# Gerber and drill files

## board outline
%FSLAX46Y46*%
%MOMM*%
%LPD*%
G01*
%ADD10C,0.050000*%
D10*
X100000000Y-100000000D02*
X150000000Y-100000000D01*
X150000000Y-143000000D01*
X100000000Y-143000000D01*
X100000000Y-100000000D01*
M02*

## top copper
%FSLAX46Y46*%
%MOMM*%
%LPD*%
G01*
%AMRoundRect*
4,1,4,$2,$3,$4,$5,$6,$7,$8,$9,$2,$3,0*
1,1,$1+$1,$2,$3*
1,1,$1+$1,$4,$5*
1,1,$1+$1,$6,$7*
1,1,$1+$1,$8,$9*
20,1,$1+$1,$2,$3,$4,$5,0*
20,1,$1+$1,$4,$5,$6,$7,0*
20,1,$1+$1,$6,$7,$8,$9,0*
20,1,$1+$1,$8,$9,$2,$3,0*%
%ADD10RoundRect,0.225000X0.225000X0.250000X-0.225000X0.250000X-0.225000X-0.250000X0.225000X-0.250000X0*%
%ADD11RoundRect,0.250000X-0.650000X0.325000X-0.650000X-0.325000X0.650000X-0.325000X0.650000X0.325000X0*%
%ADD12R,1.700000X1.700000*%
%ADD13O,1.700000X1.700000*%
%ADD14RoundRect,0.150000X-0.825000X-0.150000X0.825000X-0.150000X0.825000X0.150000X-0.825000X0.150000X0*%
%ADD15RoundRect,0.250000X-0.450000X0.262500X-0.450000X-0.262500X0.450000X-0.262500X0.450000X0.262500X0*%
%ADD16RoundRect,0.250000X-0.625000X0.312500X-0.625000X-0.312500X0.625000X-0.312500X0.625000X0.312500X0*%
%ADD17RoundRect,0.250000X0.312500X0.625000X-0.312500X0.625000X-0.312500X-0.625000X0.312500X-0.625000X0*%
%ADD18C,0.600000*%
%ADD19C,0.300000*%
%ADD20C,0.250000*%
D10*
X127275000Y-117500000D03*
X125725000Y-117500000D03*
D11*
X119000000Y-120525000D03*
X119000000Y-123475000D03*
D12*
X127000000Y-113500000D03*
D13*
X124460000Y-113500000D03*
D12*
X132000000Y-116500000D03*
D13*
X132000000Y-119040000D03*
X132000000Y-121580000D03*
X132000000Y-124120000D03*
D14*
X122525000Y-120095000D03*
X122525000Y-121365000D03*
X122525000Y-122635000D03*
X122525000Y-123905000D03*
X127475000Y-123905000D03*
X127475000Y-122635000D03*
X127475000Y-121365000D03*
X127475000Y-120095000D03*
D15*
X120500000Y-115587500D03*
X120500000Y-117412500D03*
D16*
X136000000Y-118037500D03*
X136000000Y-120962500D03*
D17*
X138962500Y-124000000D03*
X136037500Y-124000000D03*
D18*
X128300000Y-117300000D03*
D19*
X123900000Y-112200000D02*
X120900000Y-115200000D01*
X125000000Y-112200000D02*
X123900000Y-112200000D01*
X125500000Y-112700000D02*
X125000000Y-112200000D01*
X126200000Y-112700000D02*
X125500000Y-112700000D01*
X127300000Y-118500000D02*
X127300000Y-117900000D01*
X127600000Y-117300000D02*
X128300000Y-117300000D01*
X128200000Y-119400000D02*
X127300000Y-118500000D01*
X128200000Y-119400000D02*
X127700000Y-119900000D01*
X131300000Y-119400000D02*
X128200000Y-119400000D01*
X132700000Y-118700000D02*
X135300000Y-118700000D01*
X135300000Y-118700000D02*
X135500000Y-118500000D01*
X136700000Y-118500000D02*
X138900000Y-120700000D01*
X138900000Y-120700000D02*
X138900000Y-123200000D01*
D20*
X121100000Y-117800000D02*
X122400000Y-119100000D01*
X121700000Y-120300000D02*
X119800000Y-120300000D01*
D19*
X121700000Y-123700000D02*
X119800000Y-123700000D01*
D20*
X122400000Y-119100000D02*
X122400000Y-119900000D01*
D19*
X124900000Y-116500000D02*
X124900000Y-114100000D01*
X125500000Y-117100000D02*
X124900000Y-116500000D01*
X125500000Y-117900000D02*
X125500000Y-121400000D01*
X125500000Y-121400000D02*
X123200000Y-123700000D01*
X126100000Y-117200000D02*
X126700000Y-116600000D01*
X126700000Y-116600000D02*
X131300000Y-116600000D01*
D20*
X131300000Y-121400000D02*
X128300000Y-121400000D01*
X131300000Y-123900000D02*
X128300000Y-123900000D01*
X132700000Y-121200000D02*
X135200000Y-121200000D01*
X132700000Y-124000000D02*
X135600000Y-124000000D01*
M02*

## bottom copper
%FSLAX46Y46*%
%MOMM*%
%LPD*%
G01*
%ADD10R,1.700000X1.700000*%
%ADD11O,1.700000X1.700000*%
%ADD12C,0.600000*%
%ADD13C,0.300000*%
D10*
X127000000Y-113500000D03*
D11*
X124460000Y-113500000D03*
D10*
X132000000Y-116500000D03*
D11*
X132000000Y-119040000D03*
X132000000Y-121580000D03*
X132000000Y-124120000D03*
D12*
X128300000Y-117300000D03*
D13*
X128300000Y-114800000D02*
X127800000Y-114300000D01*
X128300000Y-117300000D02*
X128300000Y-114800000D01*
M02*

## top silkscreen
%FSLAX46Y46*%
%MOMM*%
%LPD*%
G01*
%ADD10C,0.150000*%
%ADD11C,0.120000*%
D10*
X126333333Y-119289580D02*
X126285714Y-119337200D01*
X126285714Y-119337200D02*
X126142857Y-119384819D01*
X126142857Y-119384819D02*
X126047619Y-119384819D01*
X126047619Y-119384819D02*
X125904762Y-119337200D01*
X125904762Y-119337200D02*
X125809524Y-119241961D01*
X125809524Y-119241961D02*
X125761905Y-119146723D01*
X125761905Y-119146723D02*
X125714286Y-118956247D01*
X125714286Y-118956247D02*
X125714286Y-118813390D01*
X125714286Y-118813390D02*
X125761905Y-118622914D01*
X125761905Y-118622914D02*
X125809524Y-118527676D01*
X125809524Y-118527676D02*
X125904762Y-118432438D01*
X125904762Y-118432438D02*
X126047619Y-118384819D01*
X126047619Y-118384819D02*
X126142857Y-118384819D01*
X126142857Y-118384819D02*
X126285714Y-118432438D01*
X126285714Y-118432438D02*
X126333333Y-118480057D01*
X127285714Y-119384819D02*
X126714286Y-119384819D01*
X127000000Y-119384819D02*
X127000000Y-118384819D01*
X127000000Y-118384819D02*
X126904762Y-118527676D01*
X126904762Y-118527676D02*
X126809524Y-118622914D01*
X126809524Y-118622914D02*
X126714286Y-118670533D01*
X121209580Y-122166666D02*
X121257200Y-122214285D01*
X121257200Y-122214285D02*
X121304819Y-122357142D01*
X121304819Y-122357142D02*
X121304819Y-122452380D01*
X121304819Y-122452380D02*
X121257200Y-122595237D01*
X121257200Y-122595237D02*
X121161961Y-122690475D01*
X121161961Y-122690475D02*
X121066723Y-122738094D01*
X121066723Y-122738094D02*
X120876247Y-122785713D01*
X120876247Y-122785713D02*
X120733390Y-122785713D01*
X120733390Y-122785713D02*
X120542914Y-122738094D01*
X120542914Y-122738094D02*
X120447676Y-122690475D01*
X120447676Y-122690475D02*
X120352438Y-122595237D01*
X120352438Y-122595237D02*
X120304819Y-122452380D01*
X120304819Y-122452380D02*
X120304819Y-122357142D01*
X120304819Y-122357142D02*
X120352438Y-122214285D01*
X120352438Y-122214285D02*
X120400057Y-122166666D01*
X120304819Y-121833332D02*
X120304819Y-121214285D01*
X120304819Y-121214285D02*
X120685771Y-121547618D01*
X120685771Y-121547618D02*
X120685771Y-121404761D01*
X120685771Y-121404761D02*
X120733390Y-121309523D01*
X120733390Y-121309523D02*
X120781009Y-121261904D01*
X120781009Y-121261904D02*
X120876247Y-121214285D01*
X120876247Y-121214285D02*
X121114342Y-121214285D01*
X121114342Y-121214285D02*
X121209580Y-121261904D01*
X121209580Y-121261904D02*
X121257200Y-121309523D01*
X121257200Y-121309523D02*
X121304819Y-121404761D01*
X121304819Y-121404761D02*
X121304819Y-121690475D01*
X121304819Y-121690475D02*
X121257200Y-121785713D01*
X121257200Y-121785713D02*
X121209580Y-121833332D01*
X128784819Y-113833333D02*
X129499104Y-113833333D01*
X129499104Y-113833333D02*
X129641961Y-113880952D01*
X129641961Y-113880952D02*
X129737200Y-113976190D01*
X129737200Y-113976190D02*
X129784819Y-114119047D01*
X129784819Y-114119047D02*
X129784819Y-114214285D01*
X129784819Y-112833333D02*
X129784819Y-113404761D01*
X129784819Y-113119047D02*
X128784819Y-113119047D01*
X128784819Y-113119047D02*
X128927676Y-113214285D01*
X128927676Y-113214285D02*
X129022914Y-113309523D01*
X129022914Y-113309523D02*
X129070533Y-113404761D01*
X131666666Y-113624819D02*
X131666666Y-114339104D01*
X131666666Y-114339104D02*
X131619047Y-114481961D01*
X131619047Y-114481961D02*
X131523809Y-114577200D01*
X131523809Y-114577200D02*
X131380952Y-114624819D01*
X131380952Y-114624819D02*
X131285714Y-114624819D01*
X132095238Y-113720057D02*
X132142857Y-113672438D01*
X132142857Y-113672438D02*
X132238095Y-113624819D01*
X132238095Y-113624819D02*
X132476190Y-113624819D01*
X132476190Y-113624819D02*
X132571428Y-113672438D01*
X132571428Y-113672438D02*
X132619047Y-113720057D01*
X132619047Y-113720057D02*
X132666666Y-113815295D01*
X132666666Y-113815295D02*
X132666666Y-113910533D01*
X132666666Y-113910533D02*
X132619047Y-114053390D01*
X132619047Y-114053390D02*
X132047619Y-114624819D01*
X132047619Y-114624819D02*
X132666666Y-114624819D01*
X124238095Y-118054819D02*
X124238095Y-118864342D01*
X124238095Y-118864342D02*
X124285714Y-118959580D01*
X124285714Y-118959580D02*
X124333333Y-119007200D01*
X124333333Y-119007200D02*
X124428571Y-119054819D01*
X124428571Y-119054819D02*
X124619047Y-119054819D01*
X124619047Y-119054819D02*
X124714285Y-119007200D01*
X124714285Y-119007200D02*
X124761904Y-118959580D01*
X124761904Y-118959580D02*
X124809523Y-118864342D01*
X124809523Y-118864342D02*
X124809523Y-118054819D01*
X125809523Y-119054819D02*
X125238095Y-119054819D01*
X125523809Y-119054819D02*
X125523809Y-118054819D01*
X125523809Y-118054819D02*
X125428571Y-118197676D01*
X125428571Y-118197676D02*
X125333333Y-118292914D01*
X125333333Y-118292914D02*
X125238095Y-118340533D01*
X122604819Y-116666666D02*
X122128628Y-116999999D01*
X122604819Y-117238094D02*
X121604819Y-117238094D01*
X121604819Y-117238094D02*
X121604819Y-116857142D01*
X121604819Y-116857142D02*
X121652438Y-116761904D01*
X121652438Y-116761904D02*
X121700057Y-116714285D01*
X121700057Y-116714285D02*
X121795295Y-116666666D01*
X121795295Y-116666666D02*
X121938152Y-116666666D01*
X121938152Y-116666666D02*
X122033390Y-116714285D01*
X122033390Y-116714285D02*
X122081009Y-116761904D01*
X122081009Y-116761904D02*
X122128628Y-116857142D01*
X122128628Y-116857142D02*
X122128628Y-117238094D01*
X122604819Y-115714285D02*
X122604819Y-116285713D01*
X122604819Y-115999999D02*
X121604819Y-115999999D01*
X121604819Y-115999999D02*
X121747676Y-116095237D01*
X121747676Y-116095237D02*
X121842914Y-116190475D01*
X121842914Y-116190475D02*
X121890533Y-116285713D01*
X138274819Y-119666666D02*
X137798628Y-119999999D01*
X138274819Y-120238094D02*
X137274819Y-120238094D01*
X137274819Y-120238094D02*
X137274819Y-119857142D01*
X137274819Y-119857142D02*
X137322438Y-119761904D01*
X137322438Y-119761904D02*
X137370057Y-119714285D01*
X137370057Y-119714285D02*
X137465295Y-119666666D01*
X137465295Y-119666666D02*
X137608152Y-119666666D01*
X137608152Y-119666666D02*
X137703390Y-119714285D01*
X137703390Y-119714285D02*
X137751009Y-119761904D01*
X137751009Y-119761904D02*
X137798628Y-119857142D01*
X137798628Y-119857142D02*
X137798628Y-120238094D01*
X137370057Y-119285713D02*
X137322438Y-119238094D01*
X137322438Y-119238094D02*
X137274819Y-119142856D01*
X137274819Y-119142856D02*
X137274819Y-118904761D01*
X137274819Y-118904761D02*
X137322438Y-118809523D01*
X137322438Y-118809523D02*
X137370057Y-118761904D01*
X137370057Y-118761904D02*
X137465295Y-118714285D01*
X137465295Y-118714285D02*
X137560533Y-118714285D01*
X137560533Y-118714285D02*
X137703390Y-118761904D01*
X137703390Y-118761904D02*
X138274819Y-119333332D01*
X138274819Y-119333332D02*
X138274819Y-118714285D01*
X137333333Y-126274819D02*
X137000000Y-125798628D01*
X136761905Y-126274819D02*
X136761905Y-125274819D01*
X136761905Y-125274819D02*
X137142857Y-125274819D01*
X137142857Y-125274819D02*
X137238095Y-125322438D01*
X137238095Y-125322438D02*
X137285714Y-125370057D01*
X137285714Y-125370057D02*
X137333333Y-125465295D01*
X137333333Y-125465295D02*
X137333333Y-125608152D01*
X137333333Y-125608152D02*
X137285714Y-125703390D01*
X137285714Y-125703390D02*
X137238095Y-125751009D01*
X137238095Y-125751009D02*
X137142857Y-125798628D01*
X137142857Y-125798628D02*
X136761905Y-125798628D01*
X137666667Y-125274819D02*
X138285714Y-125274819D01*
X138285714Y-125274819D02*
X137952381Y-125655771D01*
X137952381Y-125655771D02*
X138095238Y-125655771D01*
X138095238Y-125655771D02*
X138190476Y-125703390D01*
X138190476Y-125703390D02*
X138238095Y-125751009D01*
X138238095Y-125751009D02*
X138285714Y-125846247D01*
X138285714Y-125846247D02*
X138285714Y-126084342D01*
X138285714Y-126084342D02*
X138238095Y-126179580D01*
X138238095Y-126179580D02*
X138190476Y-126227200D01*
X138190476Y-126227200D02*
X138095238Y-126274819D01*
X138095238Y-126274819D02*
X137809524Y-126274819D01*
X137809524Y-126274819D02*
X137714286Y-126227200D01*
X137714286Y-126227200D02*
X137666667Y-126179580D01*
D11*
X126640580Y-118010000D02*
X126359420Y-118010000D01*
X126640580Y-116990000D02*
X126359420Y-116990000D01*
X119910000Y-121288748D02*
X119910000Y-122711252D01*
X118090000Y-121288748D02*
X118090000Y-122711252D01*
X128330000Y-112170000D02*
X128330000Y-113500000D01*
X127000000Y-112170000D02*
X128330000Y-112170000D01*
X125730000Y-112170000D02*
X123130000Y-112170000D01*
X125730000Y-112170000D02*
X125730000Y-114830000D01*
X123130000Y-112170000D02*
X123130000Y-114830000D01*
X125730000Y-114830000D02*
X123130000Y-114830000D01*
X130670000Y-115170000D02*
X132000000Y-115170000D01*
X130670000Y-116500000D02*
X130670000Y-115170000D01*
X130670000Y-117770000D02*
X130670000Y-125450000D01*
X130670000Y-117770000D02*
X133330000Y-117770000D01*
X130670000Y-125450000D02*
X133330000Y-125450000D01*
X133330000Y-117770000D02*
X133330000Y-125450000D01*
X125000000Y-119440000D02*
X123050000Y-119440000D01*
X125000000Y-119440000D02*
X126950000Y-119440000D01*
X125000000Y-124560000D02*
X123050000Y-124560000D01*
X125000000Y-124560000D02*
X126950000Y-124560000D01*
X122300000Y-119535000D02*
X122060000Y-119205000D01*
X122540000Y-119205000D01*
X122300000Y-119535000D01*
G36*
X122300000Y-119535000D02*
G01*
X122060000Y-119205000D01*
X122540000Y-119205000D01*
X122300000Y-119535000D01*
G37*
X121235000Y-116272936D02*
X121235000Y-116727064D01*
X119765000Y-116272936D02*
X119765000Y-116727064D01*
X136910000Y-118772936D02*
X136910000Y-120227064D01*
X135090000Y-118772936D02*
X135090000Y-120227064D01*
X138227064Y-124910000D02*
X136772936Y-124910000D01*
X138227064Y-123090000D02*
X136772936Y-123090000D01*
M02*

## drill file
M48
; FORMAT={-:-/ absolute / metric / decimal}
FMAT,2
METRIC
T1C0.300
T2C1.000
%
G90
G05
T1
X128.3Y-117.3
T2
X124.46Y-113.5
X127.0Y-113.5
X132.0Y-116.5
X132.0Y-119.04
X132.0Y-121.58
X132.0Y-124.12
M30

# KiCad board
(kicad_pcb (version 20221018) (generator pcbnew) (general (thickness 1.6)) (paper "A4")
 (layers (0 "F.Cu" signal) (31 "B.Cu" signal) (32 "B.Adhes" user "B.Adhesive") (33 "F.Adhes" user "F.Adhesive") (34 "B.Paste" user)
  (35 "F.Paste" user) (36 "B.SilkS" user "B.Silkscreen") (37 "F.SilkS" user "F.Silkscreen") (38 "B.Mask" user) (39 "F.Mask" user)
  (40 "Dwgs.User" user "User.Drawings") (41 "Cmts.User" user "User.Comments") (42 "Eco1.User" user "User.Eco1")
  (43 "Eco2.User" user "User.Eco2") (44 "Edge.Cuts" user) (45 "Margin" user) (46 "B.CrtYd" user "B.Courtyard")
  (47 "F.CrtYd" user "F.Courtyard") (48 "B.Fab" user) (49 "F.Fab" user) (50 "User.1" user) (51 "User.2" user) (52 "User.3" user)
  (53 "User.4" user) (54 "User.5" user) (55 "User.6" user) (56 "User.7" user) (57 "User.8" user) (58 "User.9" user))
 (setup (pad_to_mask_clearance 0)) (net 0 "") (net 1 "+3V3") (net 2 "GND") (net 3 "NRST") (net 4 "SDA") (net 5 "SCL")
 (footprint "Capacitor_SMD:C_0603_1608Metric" (layer "F.Cu") (at 126.5 117.5 180)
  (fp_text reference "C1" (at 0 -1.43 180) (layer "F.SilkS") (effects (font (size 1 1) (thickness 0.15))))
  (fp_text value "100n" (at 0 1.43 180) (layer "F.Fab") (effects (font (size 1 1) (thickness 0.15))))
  (fp_line (start -0.14058 -0.51) (end 0.14058 -0.51) (stroke (width 0.12) (type solid)) (layer "F.SilkS"))
  (fp_line (start -0.14058 0.51) (end 0.14058 0.51) (stroke (width 0.12) (type solid)) (layer "F.SilkS"))
  (pad "1" smd roundrect (at -0.775 0 180) (size 0.9 0.95) (layers "F.Cu" "F.Paste" "F.Mask") (roundrect_rratio 0.25) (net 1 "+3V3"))
  (pad "2" smd roundrect (at 0.775 0 180) (size 0.9 0.95) (layers "F.Cu" "F.Paste" "F.Mask") (roundrect_rratio 0.25) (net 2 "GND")))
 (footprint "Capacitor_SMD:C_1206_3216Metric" (layer "F.Cu") (at 119 122 -90)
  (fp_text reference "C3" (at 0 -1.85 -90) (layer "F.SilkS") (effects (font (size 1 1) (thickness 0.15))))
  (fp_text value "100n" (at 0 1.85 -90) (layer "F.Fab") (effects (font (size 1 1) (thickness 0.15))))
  (fp_line (start -0.711252 -0.91) (end 0.711252 -0.91) (stroke (width 0.12) (type solid)) (layer "F.SilkS"))
  (fp_line (start -0.711252 0.91) (end 0.711252 0.91) (stroke (width 0.12) (type solid)) (layer "F.SilkS"))
  (pad "1" smd roundrect (at -1.475 0 270) (size 1.15 1.8) (layers "F.Cu" "F.Paste" "F.Mask") (roundrect_rratio 0.217391) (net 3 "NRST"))
  (pad "2" smd roundrect (at 1.475 0 270) (size 1.15 1.8) (layers "F.Cu" "F.Paste" "F.Mask") (roundrect_rratio 0.217391) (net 2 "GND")))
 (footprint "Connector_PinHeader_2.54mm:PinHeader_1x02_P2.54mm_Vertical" (layer "F.Cu") (at 127 113.5 -90)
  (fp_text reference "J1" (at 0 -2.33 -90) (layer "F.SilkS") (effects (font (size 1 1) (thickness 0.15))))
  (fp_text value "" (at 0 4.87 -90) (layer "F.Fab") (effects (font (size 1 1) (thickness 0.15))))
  (fp_line (start -1.33 -1.33) (end 0 -1.33) (stroke (width 0.12) (type solid)) (layer "F.SilkS"))
  (fp_line (start -1.33 0) (end -1.33 -1.33) (stroke (width 0.12) (type solid)) (layer "F.SilkS"))
  (fp_line (start -1.33 1.27) (end -1.33 3.87) (stroke (width 0.12) (type solid)) (layer "F.SilkS"))
  (fp_line (start -1.33 1.27) (end 1.33 1.27) (stroke (width 0.12) (type solid)) (layer "F.SilkS"))
  (fp_line (start -1.33 3.87) (end 1.33 3.87) (stroke (width 0.12) (type solid)) (layer "F.SilkS"))
  (fp_line (start 1.33 1.27) (end 1.33 3.87) (stroke (width 0.12) (type solid)) (layer "F.SilkS"))
  (pad "1" thru_hole rect (at 0 0 270) (size 1.7 1.7) (drill 1) (layers "*.Cu" "*.Mask") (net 1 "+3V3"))
  (pad "2" thru_hole oval (at 0 2.54 270) (size 1.7 1.7) (drill 1) (layers "*.Cu" "*.Mask") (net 2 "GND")))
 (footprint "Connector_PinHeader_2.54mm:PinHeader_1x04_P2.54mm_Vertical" (layer "F.Cu") (at 132 116.5)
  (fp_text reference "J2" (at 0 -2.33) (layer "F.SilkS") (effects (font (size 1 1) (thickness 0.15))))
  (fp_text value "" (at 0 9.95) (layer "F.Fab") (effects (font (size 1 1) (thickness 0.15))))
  (fp_line (start -1.33 -1.33) (end 0 -1.33) (stroke (width 0.12) (type solid)) (layer "F.SilkS"))
  (fp_line (start -1.33 0) (end -1.33 -1.33) (stroke (width 0.12) (type solid)) (layer "F.SilkS"))
  (fp_line (start -1.33 1.27) (end -1.33 8.95) (stroke (width 0.12) (type solid)) (layer "F.SilkS"))
  (fp_line (start -1.33 1.27) (end 1.33 1.27) (stroke (width 0.12) (type solid)) (layer "F.SilkS"))
  (fp_line (start -1.33 8.95) (end 1.33 8.95) (stroke (width 0.12) (type solid)) (layer "F.SilkS"))
  (fp_line (start 1.33 1.27) (end 1.33 8.95) (stroke (width 0.12) (type solid)) (layer "F.SilkS"))
  (pad "1" thru_hole rect (at 0 0) (size 1.7 1.7) (drill 1) (layers "*.Cu" "*.Mask") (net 2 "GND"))
  (pad "2" thru_hole oval (at 0 2.54) (size 1.7 1.7) (drill 1) (layers "*.Cu" "*.Mask") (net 1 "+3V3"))
  (pad "3" thru_hole oval (at 0 5.08) (size 1.7 1.7) (drill 1) (layers "*.Cu" "*.Mask") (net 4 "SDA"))
  (pad "4" thru_hole oval (at 0 7.62) (size 1.7 1.7) (drill 1) (layers "*.Cu" "*.Mask") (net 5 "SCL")))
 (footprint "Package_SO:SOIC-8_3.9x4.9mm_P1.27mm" (layer "F.Cu") (at 125 122)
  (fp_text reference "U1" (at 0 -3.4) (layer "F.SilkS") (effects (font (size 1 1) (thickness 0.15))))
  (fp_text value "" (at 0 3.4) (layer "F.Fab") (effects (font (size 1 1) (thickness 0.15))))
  (fp_line (start 0 -2.56) (end -1.95 -2.56) (stroke (width 0.12) (type solid)) (layer "F.SilkS"))
  (fp_line (start 0 -2.56) (end 1.95 -2.56) (stroke (width 0.12) (type solid)) (layer "F.SilkS"))
  (fp_line (start 0 2.56) (end -1.95 2.56) (stroke (width 0.12) (type solid)) (layer "F.SilkS"))
  (fp_line (start 0 2.56) (end 1.95 2.56) (stroke (width 0.12) (type solid)) (layer "F.SilkS"))
  (fp_poly
   (pts (xy -2.7 -2.465) (xy -2.94 -2.795) (xy -2.46 -2.795) (xy -2.7 -2.465)) (stroke (width 0.12) (type solid)) (fill solid)
   (layer "F.SilkS"))
  (pad "1" smd roundrect (at -2.475 -1.905) (size 1.95 0.6) (layers "F.Cu" "F.Paste" "F.Mask") (roundrect_rratio 0.25) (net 3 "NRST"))
  (pad "2" smd roundrect (at -2.475 -0.635) (size 1.95 0.6) (layers "F.Cu" "F.Paste" "F.Mask") (roundrect_rratio 0.25))
  (pad "3" smd roundrect (at -2.475 0.635) (size 1.95 0.6) (layers "F.Cu" "F.Paste" "F.Mask") (roundrect_rratio 0.25))
  (pad "4" smd roundrect (at -2.475 1.905) (size 1.95 0.6) (layers "F.Cu" "F.Paste" "F.Mask") (roundrect_rratio 0.25) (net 2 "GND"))
  (pad "5" smd roundrect (at 2.475 1.905) (size 1.95 0.6) (layers "F.Cu" "F.Paste" "F.Mask") (roundrect_rratio 0.25) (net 5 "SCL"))
  (pad "6" smd roundrect (at 2.475 0.635) (size 1.95 0.6) (layers "F.Cu" "F.Paste" "F.Mask") (roundrect_rratio 0.25))
  (pad "7" smd roundrect (at 2.475 -0.635) (size 1.95 0.6) (layers "F.Cu" "F.Paste" "F.Mask") (roundrect_rratio 0.25) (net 4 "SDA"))
  (pad "8" smd roundrect (at 2.475 -1.905) (size 1.95 0.6) (layers "F.Cu" "F.Paste" "F.Mask") (roundrect_rratio 0.25) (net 1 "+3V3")))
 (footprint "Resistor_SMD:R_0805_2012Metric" (layer "F.Cu") (at 120.5 116.5 -90)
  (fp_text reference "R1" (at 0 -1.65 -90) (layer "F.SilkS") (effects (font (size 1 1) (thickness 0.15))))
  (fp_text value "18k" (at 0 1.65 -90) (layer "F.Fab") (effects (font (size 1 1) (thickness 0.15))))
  (fp_line (start -0.227064 -0.735) (end 0.227064 -0.735) (stroke (width 0.12) (type solid)) (layer "F.SilkS"))
  (fp_line (start -0.227064 0.735) (end 0.227064 0.735) (stroke (width 0.12) (type solid)) (layer "F.SilkS"))
  (pad "1" smd roundrect (at -0.9125 0 270) (size 1.025 1.4) (layers "F.Cu" "F.Paste" "F.Mask") (roundrect_rratio 0.243902) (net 1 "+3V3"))
  (pad "2" smd roundrect (at 0.9125 0 270) (size 1.025 1.4) (layers "F.Cu" "F.Paste" "F.Mask") (roundrect_rratio 0.243902) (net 3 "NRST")))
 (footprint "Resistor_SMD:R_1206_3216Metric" (layer "F.Cu") (at 136 119.5 -90)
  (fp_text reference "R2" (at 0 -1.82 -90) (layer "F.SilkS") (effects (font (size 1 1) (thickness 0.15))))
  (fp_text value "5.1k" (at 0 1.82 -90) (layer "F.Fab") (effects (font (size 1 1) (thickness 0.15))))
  (fp_line (start -0.727064 -0.91) (end 0.727064 -0.91) (stroke (width 0.12) (type solid)) (layer "F.SilkS"))
  (fp_line (start -0.727064 0.91) (end 0.727064 0.91) (stroke (width 0.12) (type solid)) (layer "F.SilkS"))
  (pad "1" smd roundrect (at -1.4625 0 270) (size 1.125 1.75) (layers "F.Cu" "F.Paste" "F.Mask") (roundrect_rratio 0.222222) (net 1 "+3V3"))
  (pad "2" smd roundrect (at 1.4625 0 270) (size 1.125 1.75) (layers "F.Cu" "F.Paste" "F.Mask") (roundrect_rratio 0.222222) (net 4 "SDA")))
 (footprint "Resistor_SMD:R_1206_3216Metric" (layer "F.Cu") (at 137.5 124 180)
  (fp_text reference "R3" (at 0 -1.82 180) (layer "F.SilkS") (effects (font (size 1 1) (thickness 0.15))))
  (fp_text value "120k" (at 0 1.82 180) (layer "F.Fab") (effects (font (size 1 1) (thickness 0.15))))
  (fp_line (start -0.727064 -0.91) (end 0.727064 -0.91) (stroke (width 0.12) (type solid)) (layer "F.SilkS"))
  (fp_line (start -0.727064 0.91) (end 0.727064 0.91) (stroke (width 0.12) (type solid)) (layer "F.SilkS"))
  (pad "1" smd roundrect (at -1.4625 0 180) (size 1.125 1.75) (layers "F.Cu" "F.Paste" "F.Mask") (roundrect_rratio 0.222222) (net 1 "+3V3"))
  (pad "2" smd roundrect (at 1.4625 0 180) (size 1.125 1.75) (layers "F.Cu" "F.Paste" "F.Mask") (roundrect_rratio 0.222222) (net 5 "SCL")))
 (gr_rect (start 100 100) (end 150 143) (stroke (width 0.05) (type default)) (fill none) (layer "Edge.Cuts"))
 (segment (start 123.9 112.2) (end 120.9 115.2) (width 0.3) (layer "F.Cu") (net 1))
 (segment (start 125 112.2) (end 123.9 112.2) (width 0.3) (layer "F.Cu") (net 1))
 (segment (start 125.5 112.7) (end 125 112.2) (width 0.3) (layer "F.Cu") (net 1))
 (segment (start 126.2 112.7) (end 125.5 112.7) (width 0.3) (layer "F.Cu") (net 1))
 (segment (start 127.3 118.5) (end 127.3 117.9) (width 0.3) (layer "F.Cu") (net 1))
 (segment (start 127.6 117.3) (end 128.3 117.3) (width 0.3) (layer "F.Cu") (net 1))
 (segment (start 128.2 119.4) (end 127.3 118.5) (width 0.3) (layer "F.Cu") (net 1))
 (segment (start 128.2 119.4) (end 127.7 119.9) (width 0.3) (layer "F.Cu") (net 1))
 (segment (start 131.3 119.4) (end 128.2 119.4) (width 0.3) (layer "F.Cu") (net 1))
 (segment (start 132.7 118.7) (end 135.3 118.7) (width 0.3) (layer "F.Cu") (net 1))
 (segment (start 135.3 118.7) (end 135.5 118.5) (width 0.3) (layer "F.Cu") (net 1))
 (segment (start 136.7 118.5) (end 138.9 120.7) (width 0.3) (layer "F.Cu") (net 1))
 (segment (start 138.9 120.7) (end 138.9 123.2) (width 0.3) (layer "F.Cu") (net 1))
 (via (at 128.3 117.3) (size 0.6) (drill 0.3) (layers "F.Cu" "B.Cu") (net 1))
 (segment (start 121.1 117.8) (end 122.4 119.1) (width 0.25) (layer "F.Cu") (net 3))
 (segment (start 121.7 120.3) (end 119.8 120.3) (width 0.25) (layer "F.Cu") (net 3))
 (segment (start 121.7 123.7) (end 119.8 123.7) (width 0.3) (layer "F.Cu") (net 2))
 (segment (start 122.4 119.1) (end 122.4 119.9) (width 0.25) (layer "F.Cu") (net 3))
 (segment (start 124.9 116.5) (end 124.9 114.1) (width 0.3) (layer "F.Cu") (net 2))
 (segment (start 125.5 117.1) (end 124.9 116.5) (width 0.3) (layer "F.Cu") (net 2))
 (segment (start 125.5 117.9) (end 125.5 121.4) (width 0.3) (layer "F.Cu") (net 2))
 (segment (start 125.5 121.4) (end 123.2 123.7) (width 0.3) (layer "F.Cu") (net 2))
 (segment (start 126.1 117.2) (end 126.7 116.6) (width 0.3) (layer "F.Cu") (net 2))
 (segment (start 126.7 116.6) (end 131.3 116.6) (width 0.3) (layer "F.Cu") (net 2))
 (segment (start 128.3 114.8) (end 127.8 114.3) (width 0.3) (layer "B.Cu") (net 1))
 (segment (start 128.3 117.3) (end 128.3 114.8) (width 0.3) (layer "B.Cu") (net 1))
 (segment (start 131.3 121.4) (end 128.3 121.4) (width 0.25) (layer "F.Cu") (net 4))
 (segment (start 131.3 123.9) (end 128.3 123.9) (width 0.25) (layer "F.Cu") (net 5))
 (segment (start 132.7 121.2) (end 135.2 121.2) (width 0.25) (layer "F.Cu") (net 4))
 (segment (start 132.7 124) (end 135.6 124) (width 0.25) (layer "F.Cu") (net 5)))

